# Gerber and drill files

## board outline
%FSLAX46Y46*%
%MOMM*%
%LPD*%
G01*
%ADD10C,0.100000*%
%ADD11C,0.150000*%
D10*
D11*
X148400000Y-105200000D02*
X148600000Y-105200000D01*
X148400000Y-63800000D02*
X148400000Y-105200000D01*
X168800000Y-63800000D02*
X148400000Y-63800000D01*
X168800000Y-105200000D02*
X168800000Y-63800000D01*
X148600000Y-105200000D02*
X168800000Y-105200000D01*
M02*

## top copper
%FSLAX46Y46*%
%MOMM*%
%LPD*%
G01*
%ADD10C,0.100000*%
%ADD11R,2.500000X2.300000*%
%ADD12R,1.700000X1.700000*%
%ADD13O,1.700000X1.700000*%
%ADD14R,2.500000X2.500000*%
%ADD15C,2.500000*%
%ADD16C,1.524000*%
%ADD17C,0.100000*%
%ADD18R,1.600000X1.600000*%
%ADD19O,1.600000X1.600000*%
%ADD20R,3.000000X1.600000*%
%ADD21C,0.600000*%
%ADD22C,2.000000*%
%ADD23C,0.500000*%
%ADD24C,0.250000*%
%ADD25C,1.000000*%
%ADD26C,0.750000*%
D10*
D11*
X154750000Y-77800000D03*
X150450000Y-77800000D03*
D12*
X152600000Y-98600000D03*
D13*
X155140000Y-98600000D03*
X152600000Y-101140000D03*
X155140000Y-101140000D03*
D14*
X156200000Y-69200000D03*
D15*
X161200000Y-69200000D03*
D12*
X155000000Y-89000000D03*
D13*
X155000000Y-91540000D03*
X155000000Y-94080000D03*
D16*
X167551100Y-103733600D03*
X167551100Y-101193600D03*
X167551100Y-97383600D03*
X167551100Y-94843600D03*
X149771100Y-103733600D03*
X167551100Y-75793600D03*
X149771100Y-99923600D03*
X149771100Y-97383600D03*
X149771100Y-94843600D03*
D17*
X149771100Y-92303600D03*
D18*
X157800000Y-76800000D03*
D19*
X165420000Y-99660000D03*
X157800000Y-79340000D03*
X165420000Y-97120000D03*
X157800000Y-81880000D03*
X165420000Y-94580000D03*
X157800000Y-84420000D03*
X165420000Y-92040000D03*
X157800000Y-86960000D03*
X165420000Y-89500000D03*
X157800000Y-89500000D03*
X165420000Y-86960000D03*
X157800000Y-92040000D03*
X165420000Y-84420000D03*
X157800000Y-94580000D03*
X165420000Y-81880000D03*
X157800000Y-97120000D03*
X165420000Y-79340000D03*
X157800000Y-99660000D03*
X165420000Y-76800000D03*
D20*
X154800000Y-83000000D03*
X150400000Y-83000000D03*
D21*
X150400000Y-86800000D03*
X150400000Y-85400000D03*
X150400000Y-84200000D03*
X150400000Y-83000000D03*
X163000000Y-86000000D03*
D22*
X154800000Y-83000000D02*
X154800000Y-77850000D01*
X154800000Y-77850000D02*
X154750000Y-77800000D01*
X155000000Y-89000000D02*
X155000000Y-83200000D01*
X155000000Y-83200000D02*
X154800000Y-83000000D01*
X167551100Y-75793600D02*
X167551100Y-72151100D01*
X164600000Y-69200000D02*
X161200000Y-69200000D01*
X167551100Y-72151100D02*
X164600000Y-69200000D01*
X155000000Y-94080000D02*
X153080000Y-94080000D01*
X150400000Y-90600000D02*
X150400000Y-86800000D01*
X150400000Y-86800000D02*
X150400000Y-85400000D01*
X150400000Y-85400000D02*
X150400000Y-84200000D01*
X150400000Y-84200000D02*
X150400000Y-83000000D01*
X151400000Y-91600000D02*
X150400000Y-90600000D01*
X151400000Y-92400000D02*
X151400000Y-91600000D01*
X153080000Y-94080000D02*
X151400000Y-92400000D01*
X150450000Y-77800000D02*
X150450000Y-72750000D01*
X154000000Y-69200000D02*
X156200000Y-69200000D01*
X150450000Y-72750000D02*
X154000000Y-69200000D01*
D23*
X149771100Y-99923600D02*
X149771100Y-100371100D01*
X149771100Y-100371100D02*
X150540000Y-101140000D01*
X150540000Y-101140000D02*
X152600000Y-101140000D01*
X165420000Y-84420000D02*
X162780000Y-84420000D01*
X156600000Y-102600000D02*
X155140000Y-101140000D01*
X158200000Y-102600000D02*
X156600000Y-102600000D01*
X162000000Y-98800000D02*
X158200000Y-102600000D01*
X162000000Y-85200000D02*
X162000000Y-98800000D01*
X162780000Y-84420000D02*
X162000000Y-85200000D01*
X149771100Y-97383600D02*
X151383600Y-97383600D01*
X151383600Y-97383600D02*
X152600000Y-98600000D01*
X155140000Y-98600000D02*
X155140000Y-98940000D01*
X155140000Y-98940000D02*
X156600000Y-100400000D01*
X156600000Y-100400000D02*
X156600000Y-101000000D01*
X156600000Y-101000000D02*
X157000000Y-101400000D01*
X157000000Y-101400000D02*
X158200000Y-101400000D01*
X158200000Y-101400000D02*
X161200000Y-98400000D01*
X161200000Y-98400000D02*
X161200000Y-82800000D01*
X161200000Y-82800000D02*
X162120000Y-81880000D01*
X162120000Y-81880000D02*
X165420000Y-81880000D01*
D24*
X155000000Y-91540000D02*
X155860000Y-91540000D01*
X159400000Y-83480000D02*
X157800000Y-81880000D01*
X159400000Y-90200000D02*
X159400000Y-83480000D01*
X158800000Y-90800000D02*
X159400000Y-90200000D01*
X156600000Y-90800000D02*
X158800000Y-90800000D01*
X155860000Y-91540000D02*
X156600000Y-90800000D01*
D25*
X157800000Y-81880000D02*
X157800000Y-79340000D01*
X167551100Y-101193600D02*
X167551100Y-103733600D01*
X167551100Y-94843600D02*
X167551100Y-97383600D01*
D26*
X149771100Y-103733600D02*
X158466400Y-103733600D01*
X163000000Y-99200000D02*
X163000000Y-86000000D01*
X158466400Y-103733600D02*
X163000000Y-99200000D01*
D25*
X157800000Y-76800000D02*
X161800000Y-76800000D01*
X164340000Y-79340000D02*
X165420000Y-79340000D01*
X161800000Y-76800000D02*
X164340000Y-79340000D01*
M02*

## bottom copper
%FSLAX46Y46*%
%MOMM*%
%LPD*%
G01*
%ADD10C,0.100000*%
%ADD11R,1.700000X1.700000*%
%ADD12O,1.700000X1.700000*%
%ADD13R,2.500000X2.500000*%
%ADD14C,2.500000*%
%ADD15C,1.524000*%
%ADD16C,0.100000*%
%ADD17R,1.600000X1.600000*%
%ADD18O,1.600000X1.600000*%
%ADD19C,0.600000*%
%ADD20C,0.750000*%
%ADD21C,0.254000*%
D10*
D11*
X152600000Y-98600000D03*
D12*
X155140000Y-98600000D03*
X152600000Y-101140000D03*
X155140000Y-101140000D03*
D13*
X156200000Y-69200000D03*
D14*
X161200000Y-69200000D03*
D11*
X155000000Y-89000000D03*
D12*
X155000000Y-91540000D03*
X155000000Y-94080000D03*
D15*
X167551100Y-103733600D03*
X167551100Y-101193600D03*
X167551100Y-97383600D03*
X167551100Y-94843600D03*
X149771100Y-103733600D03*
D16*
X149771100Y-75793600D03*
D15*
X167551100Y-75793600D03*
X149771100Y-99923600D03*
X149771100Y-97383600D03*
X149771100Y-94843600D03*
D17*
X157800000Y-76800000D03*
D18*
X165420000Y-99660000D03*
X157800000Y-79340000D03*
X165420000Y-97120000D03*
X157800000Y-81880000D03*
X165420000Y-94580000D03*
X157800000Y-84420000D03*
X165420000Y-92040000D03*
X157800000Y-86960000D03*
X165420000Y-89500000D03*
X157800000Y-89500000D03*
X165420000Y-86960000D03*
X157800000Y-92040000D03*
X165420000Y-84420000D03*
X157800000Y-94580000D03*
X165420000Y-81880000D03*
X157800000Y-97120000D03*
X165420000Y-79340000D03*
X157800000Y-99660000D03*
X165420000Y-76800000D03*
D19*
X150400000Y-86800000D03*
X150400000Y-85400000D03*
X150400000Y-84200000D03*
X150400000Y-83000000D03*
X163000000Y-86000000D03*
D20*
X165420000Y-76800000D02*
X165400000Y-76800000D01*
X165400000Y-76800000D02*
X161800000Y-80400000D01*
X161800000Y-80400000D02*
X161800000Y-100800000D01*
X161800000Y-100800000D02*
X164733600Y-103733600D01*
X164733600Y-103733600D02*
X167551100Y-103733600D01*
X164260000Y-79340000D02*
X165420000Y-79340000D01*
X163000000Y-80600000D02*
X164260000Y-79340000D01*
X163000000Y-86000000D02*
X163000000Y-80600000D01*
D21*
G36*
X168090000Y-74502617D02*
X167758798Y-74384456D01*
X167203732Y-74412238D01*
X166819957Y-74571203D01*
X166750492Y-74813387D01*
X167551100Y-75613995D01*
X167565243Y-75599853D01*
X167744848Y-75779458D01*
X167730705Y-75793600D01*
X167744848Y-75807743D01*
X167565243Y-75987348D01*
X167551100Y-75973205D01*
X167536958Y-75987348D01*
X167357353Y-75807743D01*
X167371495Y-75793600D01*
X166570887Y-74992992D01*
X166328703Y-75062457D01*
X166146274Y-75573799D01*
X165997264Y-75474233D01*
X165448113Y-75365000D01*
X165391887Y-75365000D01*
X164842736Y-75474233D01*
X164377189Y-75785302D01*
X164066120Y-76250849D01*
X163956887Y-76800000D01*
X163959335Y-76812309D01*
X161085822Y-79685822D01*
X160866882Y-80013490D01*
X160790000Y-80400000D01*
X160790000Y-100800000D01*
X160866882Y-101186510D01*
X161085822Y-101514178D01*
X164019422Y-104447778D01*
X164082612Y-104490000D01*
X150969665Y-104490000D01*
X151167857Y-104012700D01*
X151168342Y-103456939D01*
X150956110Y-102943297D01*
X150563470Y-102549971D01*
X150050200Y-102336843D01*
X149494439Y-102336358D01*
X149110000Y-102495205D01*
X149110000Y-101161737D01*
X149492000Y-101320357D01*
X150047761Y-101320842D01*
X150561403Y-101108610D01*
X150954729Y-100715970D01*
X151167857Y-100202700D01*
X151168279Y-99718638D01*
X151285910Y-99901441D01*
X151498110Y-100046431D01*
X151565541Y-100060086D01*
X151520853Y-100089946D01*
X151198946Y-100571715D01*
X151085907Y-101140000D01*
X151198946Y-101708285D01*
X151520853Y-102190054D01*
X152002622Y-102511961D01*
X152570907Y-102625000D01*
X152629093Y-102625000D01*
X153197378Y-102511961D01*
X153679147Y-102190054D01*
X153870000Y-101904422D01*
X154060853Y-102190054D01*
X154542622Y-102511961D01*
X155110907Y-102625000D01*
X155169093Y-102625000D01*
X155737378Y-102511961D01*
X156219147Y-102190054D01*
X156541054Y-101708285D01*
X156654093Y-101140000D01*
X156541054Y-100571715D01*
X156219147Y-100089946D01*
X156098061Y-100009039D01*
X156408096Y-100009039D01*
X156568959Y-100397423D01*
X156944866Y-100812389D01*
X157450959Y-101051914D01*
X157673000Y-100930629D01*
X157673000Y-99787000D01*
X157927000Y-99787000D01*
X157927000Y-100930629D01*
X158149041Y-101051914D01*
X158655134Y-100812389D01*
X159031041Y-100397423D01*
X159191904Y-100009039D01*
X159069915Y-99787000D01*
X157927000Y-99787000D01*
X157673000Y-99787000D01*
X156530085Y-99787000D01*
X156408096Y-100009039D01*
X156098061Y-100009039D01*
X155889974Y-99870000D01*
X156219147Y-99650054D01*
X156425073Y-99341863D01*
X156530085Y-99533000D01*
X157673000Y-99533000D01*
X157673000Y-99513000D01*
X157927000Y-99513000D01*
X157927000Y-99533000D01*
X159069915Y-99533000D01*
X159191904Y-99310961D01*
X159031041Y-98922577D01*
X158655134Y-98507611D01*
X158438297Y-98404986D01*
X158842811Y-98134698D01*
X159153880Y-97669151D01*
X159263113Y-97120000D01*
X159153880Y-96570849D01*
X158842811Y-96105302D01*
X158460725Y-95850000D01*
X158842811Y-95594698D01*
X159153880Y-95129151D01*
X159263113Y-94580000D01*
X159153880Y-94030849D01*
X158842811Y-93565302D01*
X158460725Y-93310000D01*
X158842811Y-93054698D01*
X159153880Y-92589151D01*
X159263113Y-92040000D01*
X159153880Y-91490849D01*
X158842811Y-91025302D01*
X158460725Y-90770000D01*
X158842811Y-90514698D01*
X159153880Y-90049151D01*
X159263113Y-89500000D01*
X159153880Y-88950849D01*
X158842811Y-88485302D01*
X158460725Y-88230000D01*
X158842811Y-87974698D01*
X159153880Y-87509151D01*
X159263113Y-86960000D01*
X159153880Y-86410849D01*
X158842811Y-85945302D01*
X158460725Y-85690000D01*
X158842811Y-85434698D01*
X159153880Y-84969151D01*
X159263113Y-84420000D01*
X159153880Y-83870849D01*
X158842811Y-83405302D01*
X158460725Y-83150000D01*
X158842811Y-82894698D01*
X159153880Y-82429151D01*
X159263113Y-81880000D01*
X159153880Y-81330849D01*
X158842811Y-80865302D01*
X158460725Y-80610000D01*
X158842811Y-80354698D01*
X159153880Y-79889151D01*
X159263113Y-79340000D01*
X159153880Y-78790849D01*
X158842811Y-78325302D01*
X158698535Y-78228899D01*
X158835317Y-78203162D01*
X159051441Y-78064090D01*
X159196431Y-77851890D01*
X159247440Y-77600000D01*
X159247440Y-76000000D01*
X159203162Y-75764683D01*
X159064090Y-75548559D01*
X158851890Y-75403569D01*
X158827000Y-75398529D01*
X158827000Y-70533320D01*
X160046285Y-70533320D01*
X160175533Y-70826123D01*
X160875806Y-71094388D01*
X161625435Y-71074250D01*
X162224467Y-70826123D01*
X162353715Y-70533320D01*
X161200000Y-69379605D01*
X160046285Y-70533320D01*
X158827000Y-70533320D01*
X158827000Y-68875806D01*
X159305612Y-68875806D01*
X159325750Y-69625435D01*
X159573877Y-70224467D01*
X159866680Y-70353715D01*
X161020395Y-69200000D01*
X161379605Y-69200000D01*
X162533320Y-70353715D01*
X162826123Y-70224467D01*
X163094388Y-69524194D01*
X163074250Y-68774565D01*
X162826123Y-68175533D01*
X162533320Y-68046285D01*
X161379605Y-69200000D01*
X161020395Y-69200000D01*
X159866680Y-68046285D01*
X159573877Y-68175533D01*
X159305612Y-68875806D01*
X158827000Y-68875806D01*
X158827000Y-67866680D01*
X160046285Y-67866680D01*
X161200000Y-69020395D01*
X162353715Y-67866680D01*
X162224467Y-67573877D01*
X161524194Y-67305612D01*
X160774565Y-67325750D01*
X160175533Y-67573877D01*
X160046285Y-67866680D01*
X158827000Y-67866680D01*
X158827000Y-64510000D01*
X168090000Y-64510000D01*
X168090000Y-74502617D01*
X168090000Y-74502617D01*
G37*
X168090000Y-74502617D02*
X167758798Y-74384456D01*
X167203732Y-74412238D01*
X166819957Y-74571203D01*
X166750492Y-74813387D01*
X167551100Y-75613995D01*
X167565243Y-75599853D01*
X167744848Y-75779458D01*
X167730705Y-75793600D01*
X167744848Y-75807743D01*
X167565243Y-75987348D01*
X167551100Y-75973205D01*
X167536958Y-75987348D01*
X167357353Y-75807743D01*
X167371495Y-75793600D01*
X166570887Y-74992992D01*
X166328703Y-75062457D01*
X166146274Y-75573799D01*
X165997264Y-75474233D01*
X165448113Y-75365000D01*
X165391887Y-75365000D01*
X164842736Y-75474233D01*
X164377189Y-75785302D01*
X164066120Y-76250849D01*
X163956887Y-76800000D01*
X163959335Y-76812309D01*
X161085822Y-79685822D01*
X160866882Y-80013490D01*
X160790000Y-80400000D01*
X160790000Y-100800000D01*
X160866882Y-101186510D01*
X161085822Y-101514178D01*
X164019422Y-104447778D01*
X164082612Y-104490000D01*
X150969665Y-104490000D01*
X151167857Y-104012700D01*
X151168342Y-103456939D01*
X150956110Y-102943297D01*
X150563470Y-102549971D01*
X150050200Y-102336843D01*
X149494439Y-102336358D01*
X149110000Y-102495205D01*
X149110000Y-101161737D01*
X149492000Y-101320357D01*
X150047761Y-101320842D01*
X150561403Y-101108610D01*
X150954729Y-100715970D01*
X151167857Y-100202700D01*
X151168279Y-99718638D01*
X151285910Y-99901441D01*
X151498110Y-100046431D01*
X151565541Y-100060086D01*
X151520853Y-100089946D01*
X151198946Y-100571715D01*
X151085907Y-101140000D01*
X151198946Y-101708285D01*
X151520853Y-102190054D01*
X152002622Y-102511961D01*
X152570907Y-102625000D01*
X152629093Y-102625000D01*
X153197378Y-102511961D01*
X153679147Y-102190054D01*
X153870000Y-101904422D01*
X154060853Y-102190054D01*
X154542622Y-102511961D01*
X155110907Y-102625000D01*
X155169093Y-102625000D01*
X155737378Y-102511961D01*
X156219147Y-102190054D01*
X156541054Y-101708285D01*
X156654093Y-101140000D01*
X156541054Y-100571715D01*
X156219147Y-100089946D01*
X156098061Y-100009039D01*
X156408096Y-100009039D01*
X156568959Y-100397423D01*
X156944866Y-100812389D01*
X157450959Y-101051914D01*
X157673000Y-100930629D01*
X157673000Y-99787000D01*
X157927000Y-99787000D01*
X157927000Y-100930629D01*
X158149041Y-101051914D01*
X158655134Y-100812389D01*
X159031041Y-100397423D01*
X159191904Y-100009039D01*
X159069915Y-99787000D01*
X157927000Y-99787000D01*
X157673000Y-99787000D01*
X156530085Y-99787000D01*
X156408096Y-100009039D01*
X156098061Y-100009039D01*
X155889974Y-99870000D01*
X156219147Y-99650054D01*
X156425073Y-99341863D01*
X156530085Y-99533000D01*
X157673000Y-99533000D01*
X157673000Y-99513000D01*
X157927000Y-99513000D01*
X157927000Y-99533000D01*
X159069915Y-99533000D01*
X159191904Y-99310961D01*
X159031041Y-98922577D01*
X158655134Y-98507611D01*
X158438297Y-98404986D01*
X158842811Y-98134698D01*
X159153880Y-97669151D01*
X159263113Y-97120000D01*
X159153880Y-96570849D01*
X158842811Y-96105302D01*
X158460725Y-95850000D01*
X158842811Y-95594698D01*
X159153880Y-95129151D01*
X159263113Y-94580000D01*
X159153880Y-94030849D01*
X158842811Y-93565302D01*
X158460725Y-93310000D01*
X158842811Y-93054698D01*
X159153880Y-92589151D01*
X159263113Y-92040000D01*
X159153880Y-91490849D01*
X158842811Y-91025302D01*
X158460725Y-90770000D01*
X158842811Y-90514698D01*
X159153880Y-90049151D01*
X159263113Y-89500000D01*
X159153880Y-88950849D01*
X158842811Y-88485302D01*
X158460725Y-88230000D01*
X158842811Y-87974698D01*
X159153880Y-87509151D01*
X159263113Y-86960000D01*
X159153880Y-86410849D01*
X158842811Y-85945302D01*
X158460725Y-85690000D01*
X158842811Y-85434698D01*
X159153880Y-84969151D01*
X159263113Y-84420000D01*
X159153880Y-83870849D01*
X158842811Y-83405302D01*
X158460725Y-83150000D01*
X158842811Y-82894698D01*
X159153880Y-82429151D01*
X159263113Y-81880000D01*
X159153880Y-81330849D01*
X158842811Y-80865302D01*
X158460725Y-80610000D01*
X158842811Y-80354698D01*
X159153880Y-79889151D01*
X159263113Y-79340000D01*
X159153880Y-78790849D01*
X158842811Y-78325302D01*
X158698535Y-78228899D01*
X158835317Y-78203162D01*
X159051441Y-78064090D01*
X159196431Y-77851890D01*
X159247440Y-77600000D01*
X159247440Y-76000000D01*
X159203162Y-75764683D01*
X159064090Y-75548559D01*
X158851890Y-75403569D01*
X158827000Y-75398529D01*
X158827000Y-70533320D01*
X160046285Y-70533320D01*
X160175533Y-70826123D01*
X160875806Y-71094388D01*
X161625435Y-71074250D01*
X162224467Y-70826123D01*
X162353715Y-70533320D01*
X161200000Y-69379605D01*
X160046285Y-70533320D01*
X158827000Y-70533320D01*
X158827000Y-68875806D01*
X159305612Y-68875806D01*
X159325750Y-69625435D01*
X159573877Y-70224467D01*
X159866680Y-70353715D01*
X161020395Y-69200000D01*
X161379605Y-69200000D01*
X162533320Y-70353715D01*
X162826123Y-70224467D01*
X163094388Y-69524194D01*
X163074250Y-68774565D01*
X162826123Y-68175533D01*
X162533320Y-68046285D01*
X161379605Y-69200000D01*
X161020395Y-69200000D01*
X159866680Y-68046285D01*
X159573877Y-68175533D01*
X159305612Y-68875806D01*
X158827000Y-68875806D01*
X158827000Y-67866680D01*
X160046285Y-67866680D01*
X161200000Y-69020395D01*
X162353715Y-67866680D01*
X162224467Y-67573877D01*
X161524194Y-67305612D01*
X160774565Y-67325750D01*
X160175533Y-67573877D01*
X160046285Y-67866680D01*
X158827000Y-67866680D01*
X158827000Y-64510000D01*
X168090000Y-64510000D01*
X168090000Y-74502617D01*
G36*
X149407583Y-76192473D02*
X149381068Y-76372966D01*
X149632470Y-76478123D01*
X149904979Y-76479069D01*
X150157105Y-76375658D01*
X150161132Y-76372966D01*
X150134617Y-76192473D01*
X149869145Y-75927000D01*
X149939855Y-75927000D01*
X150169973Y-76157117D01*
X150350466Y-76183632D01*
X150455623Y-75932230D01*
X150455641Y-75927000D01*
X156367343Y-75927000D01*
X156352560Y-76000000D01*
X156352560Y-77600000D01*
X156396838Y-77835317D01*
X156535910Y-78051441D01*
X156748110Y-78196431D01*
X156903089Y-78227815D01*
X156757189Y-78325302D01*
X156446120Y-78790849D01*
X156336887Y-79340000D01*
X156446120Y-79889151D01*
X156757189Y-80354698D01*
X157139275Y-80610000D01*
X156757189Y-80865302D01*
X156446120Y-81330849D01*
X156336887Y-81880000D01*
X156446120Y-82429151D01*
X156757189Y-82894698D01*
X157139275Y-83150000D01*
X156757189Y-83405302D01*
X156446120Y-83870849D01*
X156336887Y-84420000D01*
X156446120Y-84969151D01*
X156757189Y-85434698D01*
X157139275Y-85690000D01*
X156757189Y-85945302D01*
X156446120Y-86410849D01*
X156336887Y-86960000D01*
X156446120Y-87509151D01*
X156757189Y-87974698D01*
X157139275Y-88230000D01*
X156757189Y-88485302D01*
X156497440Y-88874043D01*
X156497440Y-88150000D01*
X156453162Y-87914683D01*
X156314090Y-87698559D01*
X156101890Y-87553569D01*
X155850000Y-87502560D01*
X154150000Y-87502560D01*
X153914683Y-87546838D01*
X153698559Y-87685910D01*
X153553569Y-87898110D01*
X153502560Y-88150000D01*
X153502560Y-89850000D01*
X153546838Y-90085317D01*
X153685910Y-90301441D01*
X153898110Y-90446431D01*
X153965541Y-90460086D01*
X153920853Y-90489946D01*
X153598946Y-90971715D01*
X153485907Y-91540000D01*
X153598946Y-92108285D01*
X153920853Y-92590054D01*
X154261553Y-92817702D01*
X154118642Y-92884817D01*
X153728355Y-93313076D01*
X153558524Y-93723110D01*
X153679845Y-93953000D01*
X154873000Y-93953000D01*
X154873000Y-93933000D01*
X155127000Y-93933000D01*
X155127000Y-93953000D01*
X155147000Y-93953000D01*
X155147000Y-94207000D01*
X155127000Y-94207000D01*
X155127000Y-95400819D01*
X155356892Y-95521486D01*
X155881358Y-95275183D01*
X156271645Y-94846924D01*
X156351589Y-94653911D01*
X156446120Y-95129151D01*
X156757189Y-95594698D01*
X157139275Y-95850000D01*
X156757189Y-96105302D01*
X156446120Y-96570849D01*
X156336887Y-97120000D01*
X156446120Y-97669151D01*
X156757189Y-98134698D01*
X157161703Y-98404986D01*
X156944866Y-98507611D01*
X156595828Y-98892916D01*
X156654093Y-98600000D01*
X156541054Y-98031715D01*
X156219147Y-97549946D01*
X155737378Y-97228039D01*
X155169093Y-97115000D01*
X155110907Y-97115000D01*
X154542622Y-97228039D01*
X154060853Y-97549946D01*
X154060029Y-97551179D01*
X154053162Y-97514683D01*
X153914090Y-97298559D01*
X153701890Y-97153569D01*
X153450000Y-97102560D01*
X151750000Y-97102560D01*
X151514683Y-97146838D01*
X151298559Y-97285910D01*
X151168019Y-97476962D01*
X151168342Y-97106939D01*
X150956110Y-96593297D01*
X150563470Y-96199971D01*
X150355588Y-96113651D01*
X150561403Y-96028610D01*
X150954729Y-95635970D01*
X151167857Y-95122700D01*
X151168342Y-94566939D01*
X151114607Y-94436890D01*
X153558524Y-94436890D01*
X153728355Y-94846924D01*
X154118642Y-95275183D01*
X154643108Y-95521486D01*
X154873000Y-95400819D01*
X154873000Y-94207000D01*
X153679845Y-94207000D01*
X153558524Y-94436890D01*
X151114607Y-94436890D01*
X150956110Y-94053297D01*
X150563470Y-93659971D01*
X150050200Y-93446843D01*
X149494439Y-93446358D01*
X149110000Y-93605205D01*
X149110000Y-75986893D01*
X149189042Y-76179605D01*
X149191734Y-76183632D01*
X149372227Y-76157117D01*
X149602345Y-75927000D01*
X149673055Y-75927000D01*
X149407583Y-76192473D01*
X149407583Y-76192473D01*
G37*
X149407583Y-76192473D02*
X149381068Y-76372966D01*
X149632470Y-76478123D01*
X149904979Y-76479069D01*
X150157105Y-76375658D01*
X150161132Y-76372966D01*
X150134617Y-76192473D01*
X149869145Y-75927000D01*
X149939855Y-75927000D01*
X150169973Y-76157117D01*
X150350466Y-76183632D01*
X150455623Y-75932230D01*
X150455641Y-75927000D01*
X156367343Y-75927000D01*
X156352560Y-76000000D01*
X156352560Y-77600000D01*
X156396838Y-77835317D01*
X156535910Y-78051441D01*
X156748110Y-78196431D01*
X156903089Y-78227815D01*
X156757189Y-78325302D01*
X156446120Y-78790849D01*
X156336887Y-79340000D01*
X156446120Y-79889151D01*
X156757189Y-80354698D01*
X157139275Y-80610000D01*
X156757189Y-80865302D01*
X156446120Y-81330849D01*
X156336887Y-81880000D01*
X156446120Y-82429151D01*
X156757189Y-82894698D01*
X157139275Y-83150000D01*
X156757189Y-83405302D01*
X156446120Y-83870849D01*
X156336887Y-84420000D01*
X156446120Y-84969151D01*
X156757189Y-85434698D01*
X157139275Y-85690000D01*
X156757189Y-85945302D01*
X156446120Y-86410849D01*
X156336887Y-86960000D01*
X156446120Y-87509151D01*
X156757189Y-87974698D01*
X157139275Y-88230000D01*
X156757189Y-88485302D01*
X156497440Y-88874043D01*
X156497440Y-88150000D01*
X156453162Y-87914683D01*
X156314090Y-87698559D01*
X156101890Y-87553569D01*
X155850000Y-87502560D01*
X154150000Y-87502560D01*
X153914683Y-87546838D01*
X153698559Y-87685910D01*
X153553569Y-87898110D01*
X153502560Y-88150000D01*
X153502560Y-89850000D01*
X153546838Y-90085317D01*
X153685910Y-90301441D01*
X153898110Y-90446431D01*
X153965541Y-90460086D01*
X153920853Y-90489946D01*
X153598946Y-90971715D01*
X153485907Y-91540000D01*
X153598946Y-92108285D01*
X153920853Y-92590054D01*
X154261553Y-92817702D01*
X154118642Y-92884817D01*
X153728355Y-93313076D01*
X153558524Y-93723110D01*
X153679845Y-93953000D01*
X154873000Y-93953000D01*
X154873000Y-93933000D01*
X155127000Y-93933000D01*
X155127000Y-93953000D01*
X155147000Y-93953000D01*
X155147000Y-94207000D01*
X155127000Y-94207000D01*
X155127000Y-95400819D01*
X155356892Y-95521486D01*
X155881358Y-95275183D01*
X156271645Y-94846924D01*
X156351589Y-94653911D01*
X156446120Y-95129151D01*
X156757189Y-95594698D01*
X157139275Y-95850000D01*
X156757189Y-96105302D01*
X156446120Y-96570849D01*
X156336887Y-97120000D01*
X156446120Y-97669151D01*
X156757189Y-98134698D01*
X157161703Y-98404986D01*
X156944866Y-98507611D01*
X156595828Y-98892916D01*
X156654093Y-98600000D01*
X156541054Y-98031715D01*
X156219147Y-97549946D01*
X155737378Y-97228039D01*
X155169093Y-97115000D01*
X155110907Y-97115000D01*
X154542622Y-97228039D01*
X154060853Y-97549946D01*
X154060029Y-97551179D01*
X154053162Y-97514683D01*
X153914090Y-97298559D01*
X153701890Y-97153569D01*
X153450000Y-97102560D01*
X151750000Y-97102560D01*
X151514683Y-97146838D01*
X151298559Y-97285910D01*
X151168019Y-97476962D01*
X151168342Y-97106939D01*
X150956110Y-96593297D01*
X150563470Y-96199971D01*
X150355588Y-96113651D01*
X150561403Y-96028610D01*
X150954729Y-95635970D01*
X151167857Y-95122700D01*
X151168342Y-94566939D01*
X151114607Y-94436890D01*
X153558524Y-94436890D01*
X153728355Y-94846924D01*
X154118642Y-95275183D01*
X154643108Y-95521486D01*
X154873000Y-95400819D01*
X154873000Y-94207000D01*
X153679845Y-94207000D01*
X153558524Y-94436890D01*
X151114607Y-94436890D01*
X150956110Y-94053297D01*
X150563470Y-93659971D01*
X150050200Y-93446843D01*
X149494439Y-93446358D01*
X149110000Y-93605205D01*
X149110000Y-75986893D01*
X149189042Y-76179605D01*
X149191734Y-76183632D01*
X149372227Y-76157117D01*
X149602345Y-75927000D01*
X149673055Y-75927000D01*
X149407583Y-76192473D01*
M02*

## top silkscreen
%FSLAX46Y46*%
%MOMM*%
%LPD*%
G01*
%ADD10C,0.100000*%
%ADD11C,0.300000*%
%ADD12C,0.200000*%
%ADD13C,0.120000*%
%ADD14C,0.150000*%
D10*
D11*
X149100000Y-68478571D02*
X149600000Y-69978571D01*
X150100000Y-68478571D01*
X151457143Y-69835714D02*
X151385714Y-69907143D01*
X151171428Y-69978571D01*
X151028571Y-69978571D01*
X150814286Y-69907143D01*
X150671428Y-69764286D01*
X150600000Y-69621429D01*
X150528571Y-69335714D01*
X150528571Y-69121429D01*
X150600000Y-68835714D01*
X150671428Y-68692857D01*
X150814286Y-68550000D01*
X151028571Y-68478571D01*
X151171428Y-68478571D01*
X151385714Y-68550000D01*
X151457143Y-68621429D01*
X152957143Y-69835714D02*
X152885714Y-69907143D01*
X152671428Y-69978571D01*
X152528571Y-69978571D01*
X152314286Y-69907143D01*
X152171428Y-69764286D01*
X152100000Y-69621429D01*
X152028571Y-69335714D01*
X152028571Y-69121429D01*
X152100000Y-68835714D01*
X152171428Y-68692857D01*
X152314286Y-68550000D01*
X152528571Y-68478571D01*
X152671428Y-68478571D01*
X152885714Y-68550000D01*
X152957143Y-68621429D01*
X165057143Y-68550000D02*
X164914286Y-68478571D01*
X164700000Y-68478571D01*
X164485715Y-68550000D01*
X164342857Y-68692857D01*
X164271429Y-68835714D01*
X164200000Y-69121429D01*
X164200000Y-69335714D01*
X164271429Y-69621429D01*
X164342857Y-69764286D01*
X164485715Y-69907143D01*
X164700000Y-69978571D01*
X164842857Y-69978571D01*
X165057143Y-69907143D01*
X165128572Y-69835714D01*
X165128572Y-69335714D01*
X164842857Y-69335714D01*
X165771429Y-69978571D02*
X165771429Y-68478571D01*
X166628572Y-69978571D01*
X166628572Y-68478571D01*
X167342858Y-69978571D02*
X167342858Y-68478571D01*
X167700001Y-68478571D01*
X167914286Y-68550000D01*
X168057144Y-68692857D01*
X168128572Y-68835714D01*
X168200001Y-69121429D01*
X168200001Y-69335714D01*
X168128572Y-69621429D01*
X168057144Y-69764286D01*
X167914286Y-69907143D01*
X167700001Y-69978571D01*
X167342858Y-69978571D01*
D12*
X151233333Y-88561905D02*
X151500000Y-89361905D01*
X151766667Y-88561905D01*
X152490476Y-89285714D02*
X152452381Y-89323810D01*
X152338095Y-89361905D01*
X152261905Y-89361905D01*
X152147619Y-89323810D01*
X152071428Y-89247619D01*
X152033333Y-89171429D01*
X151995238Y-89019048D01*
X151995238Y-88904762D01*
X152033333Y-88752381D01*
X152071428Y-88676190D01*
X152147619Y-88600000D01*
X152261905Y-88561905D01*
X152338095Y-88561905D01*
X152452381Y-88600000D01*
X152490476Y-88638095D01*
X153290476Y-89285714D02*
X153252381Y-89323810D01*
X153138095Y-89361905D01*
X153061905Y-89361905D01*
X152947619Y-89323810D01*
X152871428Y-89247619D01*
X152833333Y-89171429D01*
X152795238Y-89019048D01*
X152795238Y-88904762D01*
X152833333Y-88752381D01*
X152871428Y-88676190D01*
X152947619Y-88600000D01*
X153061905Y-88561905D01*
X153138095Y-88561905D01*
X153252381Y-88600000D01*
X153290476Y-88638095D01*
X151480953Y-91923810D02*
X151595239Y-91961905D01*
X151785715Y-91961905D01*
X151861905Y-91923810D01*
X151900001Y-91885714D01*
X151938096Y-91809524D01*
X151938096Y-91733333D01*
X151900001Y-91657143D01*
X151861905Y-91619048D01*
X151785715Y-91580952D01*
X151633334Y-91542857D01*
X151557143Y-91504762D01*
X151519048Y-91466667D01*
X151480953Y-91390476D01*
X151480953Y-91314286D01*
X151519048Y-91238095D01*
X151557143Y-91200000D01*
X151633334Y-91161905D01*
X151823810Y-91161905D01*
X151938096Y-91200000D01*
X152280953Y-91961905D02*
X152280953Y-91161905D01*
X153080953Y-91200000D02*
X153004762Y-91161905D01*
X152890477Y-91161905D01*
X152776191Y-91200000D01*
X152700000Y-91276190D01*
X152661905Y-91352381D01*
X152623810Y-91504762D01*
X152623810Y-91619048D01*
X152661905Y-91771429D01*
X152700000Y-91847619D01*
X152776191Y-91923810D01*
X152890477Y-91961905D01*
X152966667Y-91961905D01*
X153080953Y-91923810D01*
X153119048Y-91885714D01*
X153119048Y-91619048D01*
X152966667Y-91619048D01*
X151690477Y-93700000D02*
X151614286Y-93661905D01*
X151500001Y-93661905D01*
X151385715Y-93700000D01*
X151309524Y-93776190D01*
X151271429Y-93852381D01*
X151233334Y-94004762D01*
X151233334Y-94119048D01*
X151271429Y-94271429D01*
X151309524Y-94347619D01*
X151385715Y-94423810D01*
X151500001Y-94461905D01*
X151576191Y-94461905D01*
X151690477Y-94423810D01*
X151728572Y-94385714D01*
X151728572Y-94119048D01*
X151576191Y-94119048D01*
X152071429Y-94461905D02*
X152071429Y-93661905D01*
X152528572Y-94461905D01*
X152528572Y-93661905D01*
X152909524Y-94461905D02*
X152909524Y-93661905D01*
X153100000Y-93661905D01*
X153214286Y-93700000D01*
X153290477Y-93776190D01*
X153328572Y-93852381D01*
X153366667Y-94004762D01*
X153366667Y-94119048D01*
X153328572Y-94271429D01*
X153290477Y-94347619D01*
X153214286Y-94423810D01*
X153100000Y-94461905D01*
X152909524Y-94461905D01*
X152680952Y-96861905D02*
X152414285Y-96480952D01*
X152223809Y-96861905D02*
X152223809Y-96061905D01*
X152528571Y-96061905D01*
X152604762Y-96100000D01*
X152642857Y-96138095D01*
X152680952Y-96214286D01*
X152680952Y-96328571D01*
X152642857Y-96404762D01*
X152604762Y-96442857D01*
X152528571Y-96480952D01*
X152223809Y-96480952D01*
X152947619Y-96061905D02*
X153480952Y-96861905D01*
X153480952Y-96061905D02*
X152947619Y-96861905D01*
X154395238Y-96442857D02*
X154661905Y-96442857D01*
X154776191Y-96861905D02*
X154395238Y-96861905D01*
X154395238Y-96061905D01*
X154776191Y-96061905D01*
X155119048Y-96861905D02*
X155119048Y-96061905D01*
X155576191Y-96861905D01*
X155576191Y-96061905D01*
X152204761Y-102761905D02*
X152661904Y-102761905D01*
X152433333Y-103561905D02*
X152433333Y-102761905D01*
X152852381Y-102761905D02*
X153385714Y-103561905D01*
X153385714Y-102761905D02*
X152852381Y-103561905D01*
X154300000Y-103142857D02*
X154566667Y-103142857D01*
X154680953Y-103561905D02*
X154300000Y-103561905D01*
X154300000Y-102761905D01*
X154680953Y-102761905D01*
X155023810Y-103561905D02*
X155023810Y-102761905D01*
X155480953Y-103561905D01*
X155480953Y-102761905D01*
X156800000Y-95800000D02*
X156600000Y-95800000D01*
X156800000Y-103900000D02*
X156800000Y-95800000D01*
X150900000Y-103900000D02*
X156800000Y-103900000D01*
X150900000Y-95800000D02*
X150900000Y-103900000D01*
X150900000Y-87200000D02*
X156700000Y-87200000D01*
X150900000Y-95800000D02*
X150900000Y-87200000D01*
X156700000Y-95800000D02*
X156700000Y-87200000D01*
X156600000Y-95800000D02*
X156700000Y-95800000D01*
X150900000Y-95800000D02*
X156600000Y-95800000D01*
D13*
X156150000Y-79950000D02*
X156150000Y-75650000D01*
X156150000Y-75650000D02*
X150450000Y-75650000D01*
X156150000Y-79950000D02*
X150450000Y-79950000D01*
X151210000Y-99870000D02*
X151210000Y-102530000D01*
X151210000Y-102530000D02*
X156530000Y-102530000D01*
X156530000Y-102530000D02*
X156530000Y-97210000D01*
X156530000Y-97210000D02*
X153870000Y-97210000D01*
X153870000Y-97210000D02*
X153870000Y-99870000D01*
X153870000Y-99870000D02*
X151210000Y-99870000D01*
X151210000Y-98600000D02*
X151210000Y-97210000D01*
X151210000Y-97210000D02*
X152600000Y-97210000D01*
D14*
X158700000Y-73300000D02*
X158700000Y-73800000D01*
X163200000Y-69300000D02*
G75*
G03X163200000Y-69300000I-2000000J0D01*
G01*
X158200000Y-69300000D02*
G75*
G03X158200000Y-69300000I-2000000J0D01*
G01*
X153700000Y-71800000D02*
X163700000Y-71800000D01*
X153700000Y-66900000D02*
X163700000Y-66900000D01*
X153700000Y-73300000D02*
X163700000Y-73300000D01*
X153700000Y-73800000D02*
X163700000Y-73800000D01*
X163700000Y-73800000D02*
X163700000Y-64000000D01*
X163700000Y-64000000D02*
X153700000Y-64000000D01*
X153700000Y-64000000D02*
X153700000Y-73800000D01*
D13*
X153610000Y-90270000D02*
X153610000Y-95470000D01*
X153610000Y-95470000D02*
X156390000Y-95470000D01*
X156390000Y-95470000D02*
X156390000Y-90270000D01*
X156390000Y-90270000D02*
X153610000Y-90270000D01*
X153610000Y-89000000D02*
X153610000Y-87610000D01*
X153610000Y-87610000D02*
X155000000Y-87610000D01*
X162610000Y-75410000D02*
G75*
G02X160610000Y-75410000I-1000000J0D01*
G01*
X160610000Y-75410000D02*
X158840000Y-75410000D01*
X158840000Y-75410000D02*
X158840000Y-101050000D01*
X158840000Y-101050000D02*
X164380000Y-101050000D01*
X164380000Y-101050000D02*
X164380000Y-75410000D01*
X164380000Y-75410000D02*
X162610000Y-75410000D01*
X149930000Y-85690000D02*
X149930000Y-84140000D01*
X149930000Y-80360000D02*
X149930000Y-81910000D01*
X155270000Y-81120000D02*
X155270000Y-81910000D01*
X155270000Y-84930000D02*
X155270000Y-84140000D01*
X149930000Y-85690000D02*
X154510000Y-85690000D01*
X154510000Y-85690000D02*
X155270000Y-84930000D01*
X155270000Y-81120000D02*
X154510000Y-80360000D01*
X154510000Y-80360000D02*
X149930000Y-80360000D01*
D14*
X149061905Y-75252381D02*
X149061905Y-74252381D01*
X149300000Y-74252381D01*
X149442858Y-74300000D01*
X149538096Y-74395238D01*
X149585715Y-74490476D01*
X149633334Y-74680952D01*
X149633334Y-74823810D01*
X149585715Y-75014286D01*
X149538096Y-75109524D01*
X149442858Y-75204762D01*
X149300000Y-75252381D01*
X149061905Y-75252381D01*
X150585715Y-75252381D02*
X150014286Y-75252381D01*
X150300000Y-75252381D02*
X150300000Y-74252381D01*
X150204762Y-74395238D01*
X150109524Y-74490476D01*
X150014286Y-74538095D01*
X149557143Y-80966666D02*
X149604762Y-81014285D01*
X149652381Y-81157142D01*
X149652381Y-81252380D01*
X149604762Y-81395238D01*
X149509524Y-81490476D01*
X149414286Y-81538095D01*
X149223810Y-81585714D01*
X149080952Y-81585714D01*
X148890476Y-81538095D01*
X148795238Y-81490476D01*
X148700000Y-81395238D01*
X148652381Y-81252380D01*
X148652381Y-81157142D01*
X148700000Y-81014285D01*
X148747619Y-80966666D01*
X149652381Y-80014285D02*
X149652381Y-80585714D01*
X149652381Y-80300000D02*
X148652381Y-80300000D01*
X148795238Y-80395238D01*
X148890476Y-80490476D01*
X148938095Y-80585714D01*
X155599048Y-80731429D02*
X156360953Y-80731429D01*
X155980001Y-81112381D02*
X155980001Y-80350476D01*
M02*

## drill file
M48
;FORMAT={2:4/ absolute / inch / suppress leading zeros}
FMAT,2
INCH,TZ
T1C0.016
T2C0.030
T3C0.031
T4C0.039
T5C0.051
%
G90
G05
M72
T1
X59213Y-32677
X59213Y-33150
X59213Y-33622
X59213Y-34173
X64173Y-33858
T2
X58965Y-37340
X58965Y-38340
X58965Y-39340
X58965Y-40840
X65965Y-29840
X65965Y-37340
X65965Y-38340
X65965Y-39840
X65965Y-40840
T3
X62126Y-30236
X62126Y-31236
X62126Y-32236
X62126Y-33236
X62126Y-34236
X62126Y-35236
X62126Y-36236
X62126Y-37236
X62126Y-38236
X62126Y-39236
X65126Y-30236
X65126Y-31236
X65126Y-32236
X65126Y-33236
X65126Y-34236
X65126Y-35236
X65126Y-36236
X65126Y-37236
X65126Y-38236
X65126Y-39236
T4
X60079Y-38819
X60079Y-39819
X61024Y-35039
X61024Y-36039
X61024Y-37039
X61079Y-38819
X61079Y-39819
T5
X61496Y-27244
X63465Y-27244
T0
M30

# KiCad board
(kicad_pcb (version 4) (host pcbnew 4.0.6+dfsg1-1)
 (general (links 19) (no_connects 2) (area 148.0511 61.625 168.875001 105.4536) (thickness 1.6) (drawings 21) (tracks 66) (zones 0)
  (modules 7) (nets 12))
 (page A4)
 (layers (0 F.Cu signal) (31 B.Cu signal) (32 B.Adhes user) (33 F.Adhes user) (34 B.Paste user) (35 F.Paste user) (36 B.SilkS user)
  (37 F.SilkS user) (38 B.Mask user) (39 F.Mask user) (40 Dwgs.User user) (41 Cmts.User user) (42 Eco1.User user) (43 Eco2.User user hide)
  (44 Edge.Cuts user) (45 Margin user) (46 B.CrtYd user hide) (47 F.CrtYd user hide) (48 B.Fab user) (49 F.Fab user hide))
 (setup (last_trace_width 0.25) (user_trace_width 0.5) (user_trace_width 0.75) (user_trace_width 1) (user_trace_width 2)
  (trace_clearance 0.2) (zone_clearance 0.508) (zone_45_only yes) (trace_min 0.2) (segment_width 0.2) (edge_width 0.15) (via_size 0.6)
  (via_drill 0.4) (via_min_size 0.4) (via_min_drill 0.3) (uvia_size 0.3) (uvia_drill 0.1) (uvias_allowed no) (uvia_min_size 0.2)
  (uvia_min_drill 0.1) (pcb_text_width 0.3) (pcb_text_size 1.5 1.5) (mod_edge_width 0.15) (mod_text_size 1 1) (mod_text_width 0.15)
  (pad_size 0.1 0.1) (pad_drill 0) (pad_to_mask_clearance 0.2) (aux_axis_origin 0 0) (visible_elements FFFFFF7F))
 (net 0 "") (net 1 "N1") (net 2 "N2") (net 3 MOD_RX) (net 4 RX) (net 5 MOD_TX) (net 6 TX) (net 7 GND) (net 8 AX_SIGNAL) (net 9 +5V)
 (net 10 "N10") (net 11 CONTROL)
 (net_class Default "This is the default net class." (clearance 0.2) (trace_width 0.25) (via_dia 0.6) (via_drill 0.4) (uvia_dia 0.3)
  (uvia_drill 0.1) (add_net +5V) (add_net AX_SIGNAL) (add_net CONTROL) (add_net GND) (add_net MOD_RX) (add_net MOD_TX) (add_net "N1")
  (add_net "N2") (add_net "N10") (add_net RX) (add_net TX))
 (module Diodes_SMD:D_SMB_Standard (layer F.Cu) (at 152.6 77.8 180)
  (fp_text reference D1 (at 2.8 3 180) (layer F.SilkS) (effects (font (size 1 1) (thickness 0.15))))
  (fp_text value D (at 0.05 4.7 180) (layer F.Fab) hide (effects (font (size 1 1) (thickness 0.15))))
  (fp_line (start -3.55 -2.15) (end -3.55 2.15) (layer F.SilkS) (width 0.12))
  (fp_line (start -3.55 2.15) (end 2.15 2.15) (layer F.SilkS) (width 0.12))
  (fp_line (start -3.55 -2.15) (end 2.15 -2.15) (layer F.SilkS) (width 0.12))
  (pad 1 smd rect (at -2.15 0 180) (size 2.5 2.3) (layers F.Cu F.Paste F.Mask) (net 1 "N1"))
  (pad 2 smd rect (at 2.15 0 180) (size 2.5 2.3) (layers F.Cu F.Paste F.Mask) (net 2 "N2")))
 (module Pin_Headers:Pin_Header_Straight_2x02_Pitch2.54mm (layer F.Cu) (at 152.6 98.6)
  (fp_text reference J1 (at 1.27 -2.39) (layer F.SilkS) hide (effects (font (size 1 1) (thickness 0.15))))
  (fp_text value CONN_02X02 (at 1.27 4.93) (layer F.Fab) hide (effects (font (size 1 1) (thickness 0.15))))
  (fp_line (start -1.39 1.27) (end -1.39 3.93) (layer F.SilkS) (width 0.12))
  (fp_line (start -1.39 3.93) (end 3.93 3.93) (layer F.SilkS) (width 0.12))
  (fp_line (start 3.93 3.93) (end 3.93 -1.39) (layer F.SilkS) (width 0.12))
  (fp_line (start 3.93 -1.39) (end 1.27 -1.39) (layer F.SilkS) (width 0.12))
  (fp_line (start 1.27 -1.39) (end 1.27 1.27) (layer F.SilkS) (width 0.12))
  (fp_line (start 1.27 1.27) (end -1.39 1.27) (layer F.SilkS) (width 0.12))
  (fp_line (start -1.39 0) (end -1.39 -1.39) (layer F.SilkS) (width 0.12))
  (fp_line (start -1.39 -1.39) (end 0 -1.39) (layer F.SilkS) (width 0.12))
  (pad 1 thru_hole rect (at 0 0) (size 1.7 1.7) (drill 1) (layers *.Cu *.Mask) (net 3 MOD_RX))
  (pad 2 thru_hole oval (at 2.54 0) (size 1.7 1.7) (drill 1) (layers *.Cu *.Mask) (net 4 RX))
  (pad 3 thru_hole oval (at 0 2.54) (size 1.7 1.7) (drill 1) (layers *.Cu *.Mask) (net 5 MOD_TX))
  (pad 4 thru_hole oval (at 2.54 2.54) (size 1.7 1.7) (drill 1) (layers *.Cu *.Mask) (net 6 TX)))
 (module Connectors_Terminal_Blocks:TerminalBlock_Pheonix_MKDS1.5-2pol (layer F.Cu) (at 156.2 69.2)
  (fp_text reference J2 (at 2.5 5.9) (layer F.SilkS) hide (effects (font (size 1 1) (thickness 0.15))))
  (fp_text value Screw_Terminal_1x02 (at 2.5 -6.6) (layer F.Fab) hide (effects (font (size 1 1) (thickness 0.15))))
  (fp_line (start 2.5 4.1) (end 2.5 4.6) (layer F.SilkS) (width 0.15))
  (fp_circle (center 5 0.1) (end 3 0.1) (layer F.SilkS) (width 0.15))
  (fp_circle (center 0 0.1) (end 2 0.1) (layer F.SilkS) (width 0.15))
  (fp_line (start -2.5 2.6) (end 7.5 2.6) (layer F.SilkS) (width 0.15))
  (fp_line (start -2.5 -2.3) (end 7.5 -2.3) (layer F.SilkS) (width 0.15))
  (fp_line (start -2.5 4.1) (end 7.5 4.1) (layer F.SilkS) (width 0.15))
  (fp_line (start -2.5 4.6) (end 7.5 4.6) (layer F.SilkS) (width 0.15))
  (fp_line (start 7.5 4.6) (end 7.5 -5.2) (layer F.SilkS) (width 0.15))
  (fp_line (start 7.5 -5.2) (end -2.5 -5.2) (layer F.SilkS) (width 0.15))
  (fp_line (start -2.5 -5.2) (end -2.5 4.6) (layer F.SilkS) (width 0.15))
  (pad 1 thru_hole rect (at 0 0) (size 2.5 2.5) (drill 1.3) (layers *.Cu *.Mask) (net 2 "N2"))
  (pad 2 thru_hole circle (at 5 0) (size 2.5 2.5) (drill 1.3) (layers *.Cu *.Mask) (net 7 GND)))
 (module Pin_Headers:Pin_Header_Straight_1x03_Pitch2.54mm (layer F.Cu) (at 155 89)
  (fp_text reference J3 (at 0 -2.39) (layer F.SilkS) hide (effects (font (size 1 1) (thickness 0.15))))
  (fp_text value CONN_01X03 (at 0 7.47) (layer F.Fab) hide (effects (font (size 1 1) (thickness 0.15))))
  (fp_line (start -1.39 1.27) (end -1.39 6.47) (layer F.SilkS) (width 0.12))
  (fp_line (start -1.39 6.47) (end 1.39 6.47) (layer F.SilkS) (width 0.12))
  (fp_line (start 1.39 6.47) (end 1.39 1.27) (layer F.SilkS) (width 0.12))
  (fp_line (start 1.39 1.27) (end -1.39 1.27) (layer F.SilkS) (width 0.12))
  (fp_line (start -1.39 0) (end -1.39 -1.39) (layer F.SilkS) (width 0.12))
  (fp_line (start -1.39 -1.39) (end 0 -1.39) (layer F.SilkS) (width 0.12))
  (pad 1 thru_hole rect (at 0 0) (size 1.7 1.7) (drill 1) (layers *.Cu *.Mask) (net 1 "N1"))
  (pad 2 thru_hole oval (at 0 2.54) (size 1.7 1.7) (drill 1) (layers *.Cu *.Mask) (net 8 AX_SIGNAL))
  (pad 3 thru_hole oval (at 0 5.08) (size 1.7 1.7) (drill 1) (layers *.Cu *.Mask) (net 7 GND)))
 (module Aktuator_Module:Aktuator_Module (layer F.Cu) (at 148.5011 105.0036)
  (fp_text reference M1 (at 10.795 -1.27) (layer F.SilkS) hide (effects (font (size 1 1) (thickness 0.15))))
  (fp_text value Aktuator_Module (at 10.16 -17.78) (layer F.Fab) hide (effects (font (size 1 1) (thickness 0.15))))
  (pad 1 thru_hole circle (at 19.05 -1.27) (size 1.524 1.524) (drill 0.762) (layers *.Cu *.Mask) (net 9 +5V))
  (pad 1 thru_hole circle (at 19.05 -3.81) (size 1.524 1.524) (drill 0.762) (layers *.Cu *.Mask) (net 9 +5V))
  (pad 2 thru_hole circle (at 19.05 -7.62) (size 1.524 1.524) (drill 0.762) (layers *.Cu *.Mask) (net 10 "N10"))
  (pad 2 thru_hole circle (at 19.05 -10.16) (size 1.524 1.524) (drill 0.762) (layers *.Cu *.Mask) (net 10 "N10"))
  (pad 3 thru_hole circle (at 1.27 -1.27) (size 1.524 1.524) (drill 0.762) (layers *.Cu *.Mask) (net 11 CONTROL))
  (pad 4 smd circle (at 1.27 -29.21) (size 0.1 0.1) (layers B.Cu F.Paste F.Mask) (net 7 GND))
  (pad 4 thru_hole circle (at 19.05 -29.21) (size 1.524 1.524) (drill 0.762) (layers *.Cu *.Mask) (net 7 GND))
  (pad 6 thru_hole circle (at 1.27 -5.08) (size 1.524 1.524) (drill 0.762) (layers *.Cu *.Mask) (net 5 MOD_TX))
  (pad 7 thru_hole circle (at 1.27 -7.62) (size 1.524 1.524) (drill 0.762) (layers *.Cu *.Mask) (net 3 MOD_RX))
  (pad 8 thru_hole circle (at 1.27 -10.16) (size 1.524 1.524) (drill 0.762) (layers *.Cu *.Mask))
  (pad 9 smd circle (at 1.27 -12.7) (size 0.1 0.1) (layers F.Cu F.Paste F.Mask)))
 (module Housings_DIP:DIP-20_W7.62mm (layer F.Cu) (at 157.8 76.8)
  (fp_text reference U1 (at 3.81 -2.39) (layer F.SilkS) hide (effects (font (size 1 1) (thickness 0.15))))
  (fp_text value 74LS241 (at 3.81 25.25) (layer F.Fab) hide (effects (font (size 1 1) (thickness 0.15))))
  (fp_arc (start 3.81 -1.39) (end 2.81 -1.39) (angle -180) (layer F.SilkS) (width 0.12))
  (fp_line (start 2.81 -1.39) (end 1.04 -1.39) (layer F.SilkS) (width 0.12))
  (fp_line (start 1.04 -1.39) (end 1.04 24.25) (layer F.SilkS) (width 0.12))
  (fp_line (start 1.04 24.25) (end 6.58 24.25) (layer F.SilkS) (width 0.12))
  (fp_line (start 6.58 24.25) (end 6.58 -1.39) (layer F.SilkS) (width 0.12))
  (fp_line (start 6.58 -1.39) (end 4.81 -1.39) (layer F.SilkS) (width 0.12))
  (pad 1 thru_hole rect (at 0 0) (size 1.6 1.6) (drill 0.8) (layers *.Cu *.Mask) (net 11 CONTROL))
  (pad 11 thru_hole oval (at 7.62 22.86) (size 1.6 1.6) (drill 0.8) (layers *.Cu *.Mask))
  (pad 2 thru_hole oval (at 0 2.54) (size 1.6 1.6) (drill 0.8) (layers *.Cu *.Mask) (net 8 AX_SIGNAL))
  (pad 12 thru_hole oval (at 7.62 20.32) (size 1.6 1.6) (drill 0.8) (layers *.Cu *.Mask))
  (pad 3 thru_hole oval (at 0 5.08) (size 1.6 1.6) (drill 0.8) (layers *.Cu *.Mask) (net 8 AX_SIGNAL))
  (pad 13 thru_hole oval (at 7.62 17.78) (size 1.6 1.6) (drill 0.8) (layers *.Cu *.Mask))
  (pad 4 thru_hole oval (at 0 7.62) (size 1.6 1.6) (drill 0.8) (layers *.Cu *.Mask))
  (pad 14 thru_hole oval (at 7.62 15.24) (size 1.6 1.6) (drill 0.8) (layers *.Cu *.Mask))
  (pad 5 thru_hole oval (at 0 10.16) (size 1.6 1.6) (drill 0.8) (layers *.Cu *.Mask))
  (pad 15 thru_hole oval (at 7.62 12.7) (size 1.6 1.6) (drill 0.8) (layers *.Cu *.Mask))
  (pad 6 thru_hole oval (at 0 12.7) (size 1.6 1.6) (drill 0.8) (layers *.Cu *.Mask))
  (pad 16 thru_hole oval (at 7.62 10.16) (size 1.6 1.6) (drill 0.8) (layers *.Cu *.Mask))
  (pad 7 thru_hole oval (at 0 15.24) (size 1.6 1.6) (drill 0.8) (layers *.Cu *.Mask))
  (pad 17 thru_hole oval (at 7.62 7.62) (size 1.6 1.6) (drill 0.8) (layers *.Cu *.Mask) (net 6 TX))
  (pad 8 thru_hole oval (at 0 17.78) (size 1.6 1.6) (drill 0.8) (layers *.Cu *.Mask))
  (pad 18 thru_hole oval (at 7.62 5.08) (size 1.6 1.6) (drill 0.8) (layers *.Cu *.Mask) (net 4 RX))
  (pad 9 thru_hole oval (at 0 20.32) (size 1.6 1.6) (drill 0.8) (layers *.Cu *.Mask))
  (pad 19 thru_hole oval (at 7.62 2.54) (size 1.6 1.6) (drill 0.8) (layers *.Cu *.Mask) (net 11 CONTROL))
  (pad 10 thru_hole oval (at 0 22.86) (size 1.6 1.6) (drill 0.8) (layers *.Cu *.Mask) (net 7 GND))
  (pad 20 thru_hole oval (at 7.62 0) (size 1.6 1.6) (drill 0.8) (layers *.Cu *.Mask) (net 9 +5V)))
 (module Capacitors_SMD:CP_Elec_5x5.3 (layer F.Cu) (at 152.6 83 180)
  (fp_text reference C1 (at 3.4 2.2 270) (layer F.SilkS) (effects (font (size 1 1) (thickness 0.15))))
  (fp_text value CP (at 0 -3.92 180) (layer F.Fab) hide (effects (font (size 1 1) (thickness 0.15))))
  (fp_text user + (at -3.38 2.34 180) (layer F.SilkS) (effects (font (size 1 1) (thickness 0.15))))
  (fp_line (start 2.67 -2.69) (end 2.67 -1.14) (layer F.SilkS) (width 0.12))
  (fp_line (start 2.67 2.64) (end 2.67 1.09) (layer F.SilkS) (width 0.12))
  (fp_line (start -2.67 1.88) (end -2.67 1.09) (layer F.SilkS) (width 0.12))
  (fp_line (start -2.67 -1.93) (end -2.67 -1.14) (layer F.SilkS) (width 0.12))
  (fp_line (start 2.67 -2.69) (end -1.91 -2.69) (layer F.SilkS) (width 0.12))
  (fp_line (start -1.91 -2.69) (end -2.67 -1.93) (layer F.SilkS) (width 0.12))
  (fp_line (start -2.67 1.88) (end -1.91 2.64) (layer F.SilkS) (width 0.12))
  (fp_line (start -1.91 2.64) (end 2.67 2.64) (layer F.SilkS) (width 0.12))
  (pad 1 smd rect (at -2.2 0) (size 3 1.6) (layers F.Cu F.Paste F.Mask) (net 1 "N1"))
  (pad 2 smd rect (at 2.2 0) (size 3 1.6) (layers F.Cu F.Paste F.Mask) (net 7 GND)))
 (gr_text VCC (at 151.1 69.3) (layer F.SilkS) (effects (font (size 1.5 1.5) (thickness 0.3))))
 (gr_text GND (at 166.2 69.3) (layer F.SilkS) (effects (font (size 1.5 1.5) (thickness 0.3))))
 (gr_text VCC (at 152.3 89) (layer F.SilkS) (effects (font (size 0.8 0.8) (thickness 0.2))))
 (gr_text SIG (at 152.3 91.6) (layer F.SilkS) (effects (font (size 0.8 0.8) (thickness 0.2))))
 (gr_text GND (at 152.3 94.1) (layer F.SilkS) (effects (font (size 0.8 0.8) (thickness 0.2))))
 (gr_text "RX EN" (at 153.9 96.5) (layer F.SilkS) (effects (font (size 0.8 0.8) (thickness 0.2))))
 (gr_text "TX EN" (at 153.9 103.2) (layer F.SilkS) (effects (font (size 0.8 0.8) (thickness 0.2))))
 (gr_line (start 156.8 95.8) (end 156.6 95.8) (angle 90) (layer F.SilkS) (width 0.2))
 (gr_line (start 156.8 103.9) (end 156.8 95.8) (angle 90) (layer F.SilkS) (width 0.2))
 (gr_line (start 150.9 103.9) (end 156.8 103.9) (angle 90) (layer F.SilkS) (width 0.2))
 (gr_line (start 150.9 95.8) (end 150.9 103.9) (angle 90) (layer F.SilkS) (width 0.2))
 (gr_line (start 150.9 87.2) (end 156.7 87.2) (angle 90) (layer F.SilkS) (width 0.2))
 (gr_line (start 150.9 95.8) (end 150.9 87.2) (angle 90) (layer F.SilkS) (width 0.2))
 (gr_line (start 156.7 95.8) (end 156.7 87.2) (angle 90) (layer F.SilkS) (width 0.2))
 (gr_line (start 156.6 95.8) (end 156.7 95.8) (angle 90) (layer F.SilkS) (width 0.2))
 (gr_line (start 150.9 95.8) (end 156.6 95.8) (angle 90) (layer F.SilkS) (width 0.2))
 (gr_line (start 148.4 105.2) (end 148.6 105.2) (angle 90) (layer Edge.Cuts) (width 0.15))
 (gr_line (start 148.4 63.8) (end 148.4 105.2) (angle 90) (layer Edge.Cuts) (width 0.15))
 (gr_line (start 168.8 63.8) (end 148.4 63.8) (angle 90) (layer Edge.Cuts) (width 0.15))
 (gr_line (start 168.8 105.2) (end 168.8 63.8) (angle 90) (layer Edge.Cuts) (width 0.15))
 (gr_line (start 148.6 105.2) (end 168.8 105.2) (angle 90) (layer Edge.Cuts) (width 0.15))
 (segment (start 154.8 83) (end 154.8 77.85) (width 2) (layer F.Cu) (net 1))
 (segment (start 154.8 77.85) (end 154.75 77.8) (width 2) (layer F.Cu) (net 1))
 (segment (start 155 89) (end 155 83.2) (width 2) (layer F.Cu) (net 1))
 (segment (start 155 83.2) (end 154.8 83) (width 2) (layer F.Cu) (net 1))
 (via (at 150.4 86.8) (size 0.6) (drill 0.4) (layers F.Cu B.Cu) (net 7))
 (via (at 150.4 85.4) (size 0.6) (drill 0.4) (layers F.Cu B.Cu) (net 7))
 (via (at 150.4 84.2) (size 0.6) (drill 0.4) (layers F.Cu B.Cu) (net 7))
 (via (at 150.4 83) (size 0.6) (drill 0.4) (layers F.Cu B.Cu) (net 7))
 (segment (start 167.5511 75.7936) (end 167.5511 72.1511) (width 2) (layer F.Cu) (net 7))
 (segment (start 164.6 69.2) (end 161.2 69.2) (width 2) (layer F.Cu) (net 7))
 (segment (start 167.5511 72.1511) (end 164.6 69.2) (width 2) (layer F.Cu) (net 7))
 (segment (start 155 94.08) (end 153.08 94.08) (width 2) (layer F.Cu) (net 7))
 (segment (start 150.4 90.6) (end 150.4 86.8) (width 2) (layer F.Cu) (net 7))
 (segment (start 150.4 86.8) (end 150.4 85.4) (width 2) (layer F.Cu) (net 7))
 (segment (start 150.4 85.4) (end 150.4 84.2) (width 2) (layer F.Cu) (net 7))
 (segment (start 150.4 84.2) (end 150.4 83) (width 2) (layer F.Cu) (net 7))
 (segment (start 151.4 91.6) (end 150.4 90.6) (width 2) (layer F.Cu) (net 7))
 (segment (start 151.4 92.4) (end 151.4 91.6) (width 2) (layer F.Cu) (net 7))
 (segment (start 153.08 94.08) (end 151.4 92.4) (width 2) (layer F.Cu) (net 7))
 (segment (start 150.45 77.8) (end 150.45 72.75) (width 2) (layer F.Cu) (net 2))
 (segment (start 154 69.2) (end 156.2 69.2) (width 2) (layer F.Cu) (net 2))
 (segment (start 150.45 72.75) (end 154 69.2) (width 2) (layer F.Cu) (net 2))
 (segment (start 149.7711 99.9236) (end 149.7711 100.3711) (width 0.5) (layer F.Cu) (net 5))
 (segment (start 149.7711 100.3711) (end 150.54 101.14) (width 0.5) (layer F.Cu) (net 5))
 (segment (start 150.54 101.14) (end 152.6 101.14) (width 0.5) (layer F.Cu) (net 5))
 (segment (start 165.42 84.42) (end 162.78 84.42) (width 0.5) (layer F.Cu) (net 6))
 (segment (start 156.6 102.6) (end 155.14 101.14) (width 0.5) (layer F.Cu) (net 6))
 (segment (start 158.2 102.6) (end 156.6 102.6) (width 0.5) (layer F.Cu) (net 6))
 (segment (start 162 98.8) (end 158.2 102.6) (width 0.5) (layer F.Cu) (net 6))
 (segment (start 162 85.2) (end 162 98.8) (width 0.5) (layer F.Cu) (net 6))
 (segment (start 162.78 84.42) (end 162 85.2) (width 0.5) (layer F.Cu) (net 6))
 (segment (start 149.7711 97.3836) (end 151.3836 97.3836) (width 0.5) (layer F.Cu) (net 3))
 (segment (start 151.3836 97.3836) (end 152.6 98.6) (width 0.5) (layer F.Cu) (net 3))
 (segment (start 155.14 98.6) (end 155.14 98.94) (width 0.5) (layer F.Cu) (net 4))
 (segment (start 155.14 98.94) (end 156.6 100.4) (width 0.5) (layer F.Cu) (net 4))
 (segment (start 156.6 100.4) (end 156.6 101) (width 0.5) (layer F.Cu) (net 4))
 (segment (start 156.6 101) (end 157 101.4) (width 0.5) (layer F.Cu) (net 4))
 (segment (start 157 101.4) (end 158.2 101.4) (width 0.5) (layer F.Cu) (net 4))
 (segment (start 158.2 101.4) (end 161.2 98.4) (width 0.5) (layer F.Cu) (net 4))
 (segment (start 161.2 98.4) (end 161.2 82.8) (width 0.5) (layer F.Cu) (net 4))
 (segment (start 161.2 82.8) (end 162.12 81.88) (width 0.5) (layer F.Cu) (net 4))
 (segment (start 162.12 81.88) (end 165.42 81.88) (width 0.5) (layer F.Cu) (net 4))
 (segment (start 155 91.54) (end 155.86 91.54) (width 0.25) (layer F.Cu) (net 8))
 (segment (start 159.4 83.48) (end 157.8 81.88) (width 0.25) (layer F.Cu) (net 8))
 (segment (start 159.4 90.2) (end 159.4 83.48) (width 0.25) (layer F.Cu) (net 8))
 (segment (start 158.8 90.8) (end 159.4 90.2) (width 0.25) (layer F.Cu) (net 8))
 (segment (start 156.6 90.8) (end 158.8 90.8) (width 0.25) (layer F.Cu) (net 8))
 (segment (start 155.86 91.54) (end 156.6 90.8) (width 0.25) (layer F.Cu) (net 8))
 (segment (start 157.8 81.88) (end 157.8 79.34) (width 1) (layer F.Cu) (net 8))
 (segment (start 165.42 76.8) (end 165.4 76.8) (width 0.75) (layer B.Cu) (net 9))
 (segment (start 165.4 76.8) (end 161.8 80.4) (width 0.75) (layer B.Cu) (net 9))
 (segment (start 161.8 80.4) (end 161.8 100.8) (width 0.75) (layer B.Cu) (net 9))
 (segment (start 161.8 100.8) (end 164.7336 103.7336) (width 0.75) (layer B.Cu) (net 9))
 (segment (start 164.7336 103.7336) (end 167.5511 103.7336) (width 0.75) (layer B.Cu) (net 9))
 (segment (start 167.5511 101.1936) (end 167.5511 103.7336) (width 1) (layer F.Cu) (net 9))
 (segment (start 167.5511 94.8436) (end 167.5511 97.3836) (width 1) (layer F.Cu) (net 10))
 (segment (start 149.7711 103.7336) (end 158.4664 103.7336) (width 0.75) (layer F.Cu) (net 11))
 (segment (start 164.26 79.34) (end 165.42 79.34) (width 0.75) (layer B.Cu) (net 11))
 (segment (start 163 80.6) (end 164.26 79.34) (width 0.75) (layer B.Cu) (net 11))
 (segment (start 163 86) (end 163 80.6) (width 0.75) (layer B.Cu) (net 11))
 (via (at 163 86) (size 0.6) (drill 0.4) (layers F.Cu B.Cu) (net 11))
 (segment (start 163 99.2) (end 163 86) (width 0.75) (layer F.Cu) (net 11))
 (segment (start 158.4664 103.7336) (end 163 99.2) (width 0.75) (layer F.Cu) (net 11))
 (segment (start 157.8 76.8) (end 161.8 76.8) (width 1) (layer F.Cu) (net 11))
 (segment (start 164.34 79.34) (end 165.42 79.34) (width 1) (layer F.Cu) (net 11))
 (segment (start 161.8 76.8) (end 164.34 79.34) (width 1) (layer F.Cu) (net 11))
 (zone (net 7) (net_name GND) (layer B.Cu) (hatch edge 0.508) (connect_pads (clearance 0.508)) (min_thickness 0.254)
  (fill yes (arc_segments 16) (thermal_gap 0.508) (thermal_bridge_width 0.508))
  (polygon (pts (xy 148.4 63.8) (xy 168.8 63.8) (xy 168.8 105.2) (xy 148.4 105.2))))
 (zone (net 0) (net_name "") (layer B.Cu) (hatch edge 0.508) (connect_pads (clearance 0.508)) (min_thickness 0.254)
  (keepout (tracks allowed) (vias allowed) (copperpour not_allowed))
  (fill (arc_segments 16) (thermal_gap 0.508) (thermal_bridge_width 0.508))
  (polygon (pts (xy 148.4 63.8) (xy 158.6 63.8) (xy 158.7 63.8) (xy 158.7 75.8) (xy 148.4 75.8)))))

